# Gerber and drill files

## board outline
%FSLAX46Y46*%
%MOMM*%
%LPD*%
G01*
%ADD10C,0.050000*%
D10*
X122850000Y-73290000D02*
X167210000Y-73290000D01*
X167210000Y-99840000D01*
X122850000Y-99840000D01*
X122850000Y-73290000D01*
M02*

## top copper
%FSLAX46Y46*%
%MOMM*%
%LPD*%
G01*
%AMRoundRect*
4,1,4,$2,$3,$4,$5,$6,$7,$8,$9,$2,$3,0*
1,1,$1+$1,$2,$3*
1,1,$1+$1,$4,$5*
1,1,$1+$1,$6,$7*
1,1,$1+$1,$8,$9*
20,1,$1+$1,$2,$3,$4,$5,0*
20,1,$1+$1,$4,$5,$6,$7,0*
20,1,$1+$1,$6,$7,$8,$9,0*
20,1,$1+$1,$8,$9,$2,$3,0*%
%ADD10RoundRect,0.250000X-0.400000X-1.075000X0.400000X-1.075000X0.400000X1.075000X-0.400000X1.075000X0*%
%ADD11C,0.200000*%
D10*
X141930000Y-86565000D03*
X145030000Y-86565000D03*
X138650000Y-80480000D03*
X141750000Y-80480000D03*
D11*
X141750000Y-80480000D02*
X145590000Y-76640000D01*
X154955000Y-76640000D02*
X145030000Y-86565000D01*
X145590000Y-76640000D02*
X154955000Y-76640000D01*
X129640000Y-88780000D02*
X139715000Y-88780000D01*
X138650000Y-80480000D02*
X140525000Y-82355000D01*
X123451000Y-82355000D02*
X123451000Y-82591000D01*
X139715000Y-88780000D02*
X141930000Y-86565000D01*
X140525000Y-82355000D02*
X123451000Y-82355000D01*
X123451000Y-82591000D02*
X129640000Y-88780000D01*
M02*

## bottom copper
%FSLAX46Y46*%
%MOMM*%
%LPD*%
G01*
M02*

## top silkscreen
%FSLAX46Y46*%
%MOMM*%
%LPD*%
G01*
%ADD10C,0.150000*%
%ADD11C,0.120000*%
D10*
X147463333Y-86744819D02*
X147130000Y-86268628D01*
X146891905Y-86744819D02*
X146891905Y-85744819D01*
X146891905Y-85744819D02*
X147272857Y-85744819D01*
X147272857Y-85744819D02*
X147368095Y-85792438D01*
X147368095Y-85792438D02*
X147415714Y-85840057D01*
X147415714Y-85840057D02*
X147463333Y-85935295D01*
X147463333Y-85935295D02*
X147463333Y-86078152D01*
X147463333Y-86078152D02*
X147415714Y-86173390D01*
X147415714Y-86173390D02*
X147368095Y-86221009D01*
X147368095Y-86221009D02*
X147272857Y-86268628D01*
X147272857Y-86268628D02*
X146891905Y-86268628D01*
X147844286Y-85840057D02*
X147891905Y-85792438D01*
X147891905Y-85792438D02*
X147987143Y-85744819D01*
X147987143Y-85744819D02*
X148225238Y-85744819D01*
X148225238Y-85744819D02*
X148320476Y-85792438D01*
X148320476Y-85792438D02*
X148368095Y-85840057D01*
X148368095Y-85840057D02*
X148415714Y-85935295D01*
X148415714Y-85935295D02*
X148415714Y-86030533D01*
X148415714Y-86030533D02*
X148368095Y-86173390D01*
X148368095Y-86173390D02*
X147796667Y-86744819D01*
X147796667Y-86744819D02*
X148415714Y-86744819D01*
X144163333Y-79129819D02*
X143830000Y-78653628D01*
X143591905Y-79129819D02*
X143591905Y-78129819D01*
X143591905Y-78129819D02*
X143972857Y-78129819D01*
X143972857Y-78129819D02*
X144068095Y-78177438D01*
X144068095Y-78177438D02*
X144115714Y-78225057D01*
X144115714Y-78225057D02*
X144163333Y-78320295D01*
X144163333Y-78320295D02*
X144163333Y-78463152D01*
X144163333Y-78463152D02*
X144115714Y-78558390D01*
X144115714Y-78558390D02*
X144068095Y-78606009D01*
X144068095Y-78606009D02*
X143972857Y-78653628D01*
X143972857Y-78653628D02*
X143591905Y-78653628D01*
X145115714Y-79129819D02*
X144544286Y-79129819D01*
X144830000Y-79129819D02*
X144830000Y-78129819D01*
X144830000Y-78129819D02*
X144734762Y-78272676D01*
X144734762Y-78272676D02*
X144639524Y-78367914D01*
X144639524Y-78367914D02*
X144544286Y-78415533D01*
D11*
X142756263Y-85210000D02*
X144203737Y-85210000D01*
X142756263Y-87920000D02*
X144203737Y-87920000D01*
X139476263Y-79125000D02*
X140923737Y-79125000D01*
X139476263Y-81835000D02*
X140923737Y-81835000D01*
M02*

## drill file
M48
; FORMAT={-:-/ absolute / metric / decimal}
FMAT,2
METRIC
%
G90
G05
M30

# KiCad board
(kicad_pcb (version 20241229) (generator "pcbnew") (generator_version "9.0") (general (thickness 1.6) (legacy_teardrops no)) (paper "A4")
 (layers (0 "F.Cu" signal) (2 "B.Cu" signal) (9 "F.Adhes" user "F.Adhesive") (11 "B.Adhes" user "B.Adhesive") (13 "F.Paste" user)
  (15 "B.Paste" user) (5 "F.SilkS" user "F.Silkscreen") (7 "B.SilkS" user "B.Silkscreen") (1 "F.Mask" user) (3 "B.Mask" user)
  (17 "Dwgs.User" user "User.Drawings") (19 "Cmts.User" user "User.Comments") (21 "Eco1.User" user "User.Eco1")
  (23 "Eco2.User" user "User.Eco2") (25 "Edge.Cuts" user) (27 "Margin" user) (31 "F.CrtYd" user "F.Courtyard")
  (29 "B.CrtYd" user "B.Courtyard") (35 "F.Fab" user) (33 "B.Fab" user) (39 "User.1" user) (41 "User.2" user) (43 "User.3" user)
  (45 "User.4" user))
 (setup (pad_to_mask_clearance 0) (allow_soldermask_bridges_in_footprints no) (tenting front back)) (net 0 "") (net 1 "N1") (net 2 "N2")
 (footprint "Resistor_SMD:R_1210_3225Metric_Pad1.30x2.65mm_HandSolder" (layer "F.Cu") (at 143.48 86.565)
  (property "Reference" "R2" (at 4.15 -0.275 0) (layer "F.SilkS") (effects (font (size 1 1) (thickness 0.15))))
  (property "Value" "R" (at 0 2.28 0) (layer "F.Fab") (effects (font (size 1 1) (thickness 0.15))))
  (fp_line (start -0.723737 -1.355) (end 0.723737 -1.355) (stroke (width 0.12) (type solid)) (layer "F.SilkS"))
  (fp_line (start -0.723737 1.355) (end 0.723737 1.355) (stroke (width 0.12) (type solid)) (layer "F.SilkS"))
  (pad "1" smd roundrect (at -1.55 0) (size 1.3 2.65) (layers "F.Cu" "F.Mask" "F.Paste") (roundrect_rratio 0.192308) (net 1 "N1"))
  (pad "2" smd roundrect (at 1.55 0) (size 1.3 2.65) (layers "F.Cu" "F.Mask" "F.Paste") (roundrect_rratio 0.192308) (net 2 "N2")))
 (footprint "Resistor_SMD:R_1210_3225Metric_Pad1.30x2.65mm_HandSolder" (layer "F.Cu") (at 140.2 80.48)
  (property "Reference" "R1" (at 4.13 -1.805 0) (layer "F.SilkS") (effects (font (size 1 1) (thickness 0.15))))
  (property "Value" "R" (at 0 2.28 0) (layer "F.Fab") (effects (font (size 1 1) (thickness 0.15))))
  (fp_line (start -0.723737 -1.355) (end 0.723737 -1.355) (stroke (width 0.12) (type solid)) (layer "F.SilkS"))
  (fp_line (start -0.723737 1.355) (end 0.723737 1.355) (stroke (width 0.12) (type solid)) (layer "F.SilkS"))
  (pad "1" smd roundrect (at -1.55 0) (size 1.3 2.65) (layers "F.Cu" "F.Mask" "F.Paste") (roundrect_rratio 0.192308) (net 1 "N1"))
  (pad "2" smd roundrect (at 1.55 0) (size 1.3 2.65) (layers "F.Cu" "F.Mask" "F.Paste") (roundrect_rratio 0.192308) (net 2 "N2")))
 (gr_rect (start 122.85 73.29) (end 167.21 99.84) (stroke (width 0.05) (type default)) (fill no) (layer "Edge.Cuts"))
 (segment (start 141.75 80.48) (end 145.59 76.64) (width 0.2) (layer "F.Cu") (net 2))
 (segment (start 154.955 76.64) (end 145.03 86.565) (width 0.2) (layer "F.Cu") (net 2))
 (segment (start 145.59 76.64) (end 154.955 76.64) (width 0.2) (layer "F.Cu") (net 2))
 (segment (start 129.64 88.78) (end 139.715 88.78) (width 0.2) (layer "F.Cu") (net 1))
 (segment (start 138.65 80.48) (end 140.525 82.355) (width 0.2) (layer "F.Cu") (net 1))
 (segment (start 123.451 82.355) (end 123.451 82.591) (width 0.2) (layer "F.Cu") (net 1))
 (segment (start 139.715 88.78) (end 141.93 86.565) (width 0.2) (layer "F.Cu") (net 1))
 (segment (start 140.525 82.355) (end 123.451 82.355) (width 0.2) (layer "F.Cu") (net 1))
 (segment (start 123.451 82.591) (end 129.64 88.78) (width 0.2) (layer "F.Cu") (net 1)))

